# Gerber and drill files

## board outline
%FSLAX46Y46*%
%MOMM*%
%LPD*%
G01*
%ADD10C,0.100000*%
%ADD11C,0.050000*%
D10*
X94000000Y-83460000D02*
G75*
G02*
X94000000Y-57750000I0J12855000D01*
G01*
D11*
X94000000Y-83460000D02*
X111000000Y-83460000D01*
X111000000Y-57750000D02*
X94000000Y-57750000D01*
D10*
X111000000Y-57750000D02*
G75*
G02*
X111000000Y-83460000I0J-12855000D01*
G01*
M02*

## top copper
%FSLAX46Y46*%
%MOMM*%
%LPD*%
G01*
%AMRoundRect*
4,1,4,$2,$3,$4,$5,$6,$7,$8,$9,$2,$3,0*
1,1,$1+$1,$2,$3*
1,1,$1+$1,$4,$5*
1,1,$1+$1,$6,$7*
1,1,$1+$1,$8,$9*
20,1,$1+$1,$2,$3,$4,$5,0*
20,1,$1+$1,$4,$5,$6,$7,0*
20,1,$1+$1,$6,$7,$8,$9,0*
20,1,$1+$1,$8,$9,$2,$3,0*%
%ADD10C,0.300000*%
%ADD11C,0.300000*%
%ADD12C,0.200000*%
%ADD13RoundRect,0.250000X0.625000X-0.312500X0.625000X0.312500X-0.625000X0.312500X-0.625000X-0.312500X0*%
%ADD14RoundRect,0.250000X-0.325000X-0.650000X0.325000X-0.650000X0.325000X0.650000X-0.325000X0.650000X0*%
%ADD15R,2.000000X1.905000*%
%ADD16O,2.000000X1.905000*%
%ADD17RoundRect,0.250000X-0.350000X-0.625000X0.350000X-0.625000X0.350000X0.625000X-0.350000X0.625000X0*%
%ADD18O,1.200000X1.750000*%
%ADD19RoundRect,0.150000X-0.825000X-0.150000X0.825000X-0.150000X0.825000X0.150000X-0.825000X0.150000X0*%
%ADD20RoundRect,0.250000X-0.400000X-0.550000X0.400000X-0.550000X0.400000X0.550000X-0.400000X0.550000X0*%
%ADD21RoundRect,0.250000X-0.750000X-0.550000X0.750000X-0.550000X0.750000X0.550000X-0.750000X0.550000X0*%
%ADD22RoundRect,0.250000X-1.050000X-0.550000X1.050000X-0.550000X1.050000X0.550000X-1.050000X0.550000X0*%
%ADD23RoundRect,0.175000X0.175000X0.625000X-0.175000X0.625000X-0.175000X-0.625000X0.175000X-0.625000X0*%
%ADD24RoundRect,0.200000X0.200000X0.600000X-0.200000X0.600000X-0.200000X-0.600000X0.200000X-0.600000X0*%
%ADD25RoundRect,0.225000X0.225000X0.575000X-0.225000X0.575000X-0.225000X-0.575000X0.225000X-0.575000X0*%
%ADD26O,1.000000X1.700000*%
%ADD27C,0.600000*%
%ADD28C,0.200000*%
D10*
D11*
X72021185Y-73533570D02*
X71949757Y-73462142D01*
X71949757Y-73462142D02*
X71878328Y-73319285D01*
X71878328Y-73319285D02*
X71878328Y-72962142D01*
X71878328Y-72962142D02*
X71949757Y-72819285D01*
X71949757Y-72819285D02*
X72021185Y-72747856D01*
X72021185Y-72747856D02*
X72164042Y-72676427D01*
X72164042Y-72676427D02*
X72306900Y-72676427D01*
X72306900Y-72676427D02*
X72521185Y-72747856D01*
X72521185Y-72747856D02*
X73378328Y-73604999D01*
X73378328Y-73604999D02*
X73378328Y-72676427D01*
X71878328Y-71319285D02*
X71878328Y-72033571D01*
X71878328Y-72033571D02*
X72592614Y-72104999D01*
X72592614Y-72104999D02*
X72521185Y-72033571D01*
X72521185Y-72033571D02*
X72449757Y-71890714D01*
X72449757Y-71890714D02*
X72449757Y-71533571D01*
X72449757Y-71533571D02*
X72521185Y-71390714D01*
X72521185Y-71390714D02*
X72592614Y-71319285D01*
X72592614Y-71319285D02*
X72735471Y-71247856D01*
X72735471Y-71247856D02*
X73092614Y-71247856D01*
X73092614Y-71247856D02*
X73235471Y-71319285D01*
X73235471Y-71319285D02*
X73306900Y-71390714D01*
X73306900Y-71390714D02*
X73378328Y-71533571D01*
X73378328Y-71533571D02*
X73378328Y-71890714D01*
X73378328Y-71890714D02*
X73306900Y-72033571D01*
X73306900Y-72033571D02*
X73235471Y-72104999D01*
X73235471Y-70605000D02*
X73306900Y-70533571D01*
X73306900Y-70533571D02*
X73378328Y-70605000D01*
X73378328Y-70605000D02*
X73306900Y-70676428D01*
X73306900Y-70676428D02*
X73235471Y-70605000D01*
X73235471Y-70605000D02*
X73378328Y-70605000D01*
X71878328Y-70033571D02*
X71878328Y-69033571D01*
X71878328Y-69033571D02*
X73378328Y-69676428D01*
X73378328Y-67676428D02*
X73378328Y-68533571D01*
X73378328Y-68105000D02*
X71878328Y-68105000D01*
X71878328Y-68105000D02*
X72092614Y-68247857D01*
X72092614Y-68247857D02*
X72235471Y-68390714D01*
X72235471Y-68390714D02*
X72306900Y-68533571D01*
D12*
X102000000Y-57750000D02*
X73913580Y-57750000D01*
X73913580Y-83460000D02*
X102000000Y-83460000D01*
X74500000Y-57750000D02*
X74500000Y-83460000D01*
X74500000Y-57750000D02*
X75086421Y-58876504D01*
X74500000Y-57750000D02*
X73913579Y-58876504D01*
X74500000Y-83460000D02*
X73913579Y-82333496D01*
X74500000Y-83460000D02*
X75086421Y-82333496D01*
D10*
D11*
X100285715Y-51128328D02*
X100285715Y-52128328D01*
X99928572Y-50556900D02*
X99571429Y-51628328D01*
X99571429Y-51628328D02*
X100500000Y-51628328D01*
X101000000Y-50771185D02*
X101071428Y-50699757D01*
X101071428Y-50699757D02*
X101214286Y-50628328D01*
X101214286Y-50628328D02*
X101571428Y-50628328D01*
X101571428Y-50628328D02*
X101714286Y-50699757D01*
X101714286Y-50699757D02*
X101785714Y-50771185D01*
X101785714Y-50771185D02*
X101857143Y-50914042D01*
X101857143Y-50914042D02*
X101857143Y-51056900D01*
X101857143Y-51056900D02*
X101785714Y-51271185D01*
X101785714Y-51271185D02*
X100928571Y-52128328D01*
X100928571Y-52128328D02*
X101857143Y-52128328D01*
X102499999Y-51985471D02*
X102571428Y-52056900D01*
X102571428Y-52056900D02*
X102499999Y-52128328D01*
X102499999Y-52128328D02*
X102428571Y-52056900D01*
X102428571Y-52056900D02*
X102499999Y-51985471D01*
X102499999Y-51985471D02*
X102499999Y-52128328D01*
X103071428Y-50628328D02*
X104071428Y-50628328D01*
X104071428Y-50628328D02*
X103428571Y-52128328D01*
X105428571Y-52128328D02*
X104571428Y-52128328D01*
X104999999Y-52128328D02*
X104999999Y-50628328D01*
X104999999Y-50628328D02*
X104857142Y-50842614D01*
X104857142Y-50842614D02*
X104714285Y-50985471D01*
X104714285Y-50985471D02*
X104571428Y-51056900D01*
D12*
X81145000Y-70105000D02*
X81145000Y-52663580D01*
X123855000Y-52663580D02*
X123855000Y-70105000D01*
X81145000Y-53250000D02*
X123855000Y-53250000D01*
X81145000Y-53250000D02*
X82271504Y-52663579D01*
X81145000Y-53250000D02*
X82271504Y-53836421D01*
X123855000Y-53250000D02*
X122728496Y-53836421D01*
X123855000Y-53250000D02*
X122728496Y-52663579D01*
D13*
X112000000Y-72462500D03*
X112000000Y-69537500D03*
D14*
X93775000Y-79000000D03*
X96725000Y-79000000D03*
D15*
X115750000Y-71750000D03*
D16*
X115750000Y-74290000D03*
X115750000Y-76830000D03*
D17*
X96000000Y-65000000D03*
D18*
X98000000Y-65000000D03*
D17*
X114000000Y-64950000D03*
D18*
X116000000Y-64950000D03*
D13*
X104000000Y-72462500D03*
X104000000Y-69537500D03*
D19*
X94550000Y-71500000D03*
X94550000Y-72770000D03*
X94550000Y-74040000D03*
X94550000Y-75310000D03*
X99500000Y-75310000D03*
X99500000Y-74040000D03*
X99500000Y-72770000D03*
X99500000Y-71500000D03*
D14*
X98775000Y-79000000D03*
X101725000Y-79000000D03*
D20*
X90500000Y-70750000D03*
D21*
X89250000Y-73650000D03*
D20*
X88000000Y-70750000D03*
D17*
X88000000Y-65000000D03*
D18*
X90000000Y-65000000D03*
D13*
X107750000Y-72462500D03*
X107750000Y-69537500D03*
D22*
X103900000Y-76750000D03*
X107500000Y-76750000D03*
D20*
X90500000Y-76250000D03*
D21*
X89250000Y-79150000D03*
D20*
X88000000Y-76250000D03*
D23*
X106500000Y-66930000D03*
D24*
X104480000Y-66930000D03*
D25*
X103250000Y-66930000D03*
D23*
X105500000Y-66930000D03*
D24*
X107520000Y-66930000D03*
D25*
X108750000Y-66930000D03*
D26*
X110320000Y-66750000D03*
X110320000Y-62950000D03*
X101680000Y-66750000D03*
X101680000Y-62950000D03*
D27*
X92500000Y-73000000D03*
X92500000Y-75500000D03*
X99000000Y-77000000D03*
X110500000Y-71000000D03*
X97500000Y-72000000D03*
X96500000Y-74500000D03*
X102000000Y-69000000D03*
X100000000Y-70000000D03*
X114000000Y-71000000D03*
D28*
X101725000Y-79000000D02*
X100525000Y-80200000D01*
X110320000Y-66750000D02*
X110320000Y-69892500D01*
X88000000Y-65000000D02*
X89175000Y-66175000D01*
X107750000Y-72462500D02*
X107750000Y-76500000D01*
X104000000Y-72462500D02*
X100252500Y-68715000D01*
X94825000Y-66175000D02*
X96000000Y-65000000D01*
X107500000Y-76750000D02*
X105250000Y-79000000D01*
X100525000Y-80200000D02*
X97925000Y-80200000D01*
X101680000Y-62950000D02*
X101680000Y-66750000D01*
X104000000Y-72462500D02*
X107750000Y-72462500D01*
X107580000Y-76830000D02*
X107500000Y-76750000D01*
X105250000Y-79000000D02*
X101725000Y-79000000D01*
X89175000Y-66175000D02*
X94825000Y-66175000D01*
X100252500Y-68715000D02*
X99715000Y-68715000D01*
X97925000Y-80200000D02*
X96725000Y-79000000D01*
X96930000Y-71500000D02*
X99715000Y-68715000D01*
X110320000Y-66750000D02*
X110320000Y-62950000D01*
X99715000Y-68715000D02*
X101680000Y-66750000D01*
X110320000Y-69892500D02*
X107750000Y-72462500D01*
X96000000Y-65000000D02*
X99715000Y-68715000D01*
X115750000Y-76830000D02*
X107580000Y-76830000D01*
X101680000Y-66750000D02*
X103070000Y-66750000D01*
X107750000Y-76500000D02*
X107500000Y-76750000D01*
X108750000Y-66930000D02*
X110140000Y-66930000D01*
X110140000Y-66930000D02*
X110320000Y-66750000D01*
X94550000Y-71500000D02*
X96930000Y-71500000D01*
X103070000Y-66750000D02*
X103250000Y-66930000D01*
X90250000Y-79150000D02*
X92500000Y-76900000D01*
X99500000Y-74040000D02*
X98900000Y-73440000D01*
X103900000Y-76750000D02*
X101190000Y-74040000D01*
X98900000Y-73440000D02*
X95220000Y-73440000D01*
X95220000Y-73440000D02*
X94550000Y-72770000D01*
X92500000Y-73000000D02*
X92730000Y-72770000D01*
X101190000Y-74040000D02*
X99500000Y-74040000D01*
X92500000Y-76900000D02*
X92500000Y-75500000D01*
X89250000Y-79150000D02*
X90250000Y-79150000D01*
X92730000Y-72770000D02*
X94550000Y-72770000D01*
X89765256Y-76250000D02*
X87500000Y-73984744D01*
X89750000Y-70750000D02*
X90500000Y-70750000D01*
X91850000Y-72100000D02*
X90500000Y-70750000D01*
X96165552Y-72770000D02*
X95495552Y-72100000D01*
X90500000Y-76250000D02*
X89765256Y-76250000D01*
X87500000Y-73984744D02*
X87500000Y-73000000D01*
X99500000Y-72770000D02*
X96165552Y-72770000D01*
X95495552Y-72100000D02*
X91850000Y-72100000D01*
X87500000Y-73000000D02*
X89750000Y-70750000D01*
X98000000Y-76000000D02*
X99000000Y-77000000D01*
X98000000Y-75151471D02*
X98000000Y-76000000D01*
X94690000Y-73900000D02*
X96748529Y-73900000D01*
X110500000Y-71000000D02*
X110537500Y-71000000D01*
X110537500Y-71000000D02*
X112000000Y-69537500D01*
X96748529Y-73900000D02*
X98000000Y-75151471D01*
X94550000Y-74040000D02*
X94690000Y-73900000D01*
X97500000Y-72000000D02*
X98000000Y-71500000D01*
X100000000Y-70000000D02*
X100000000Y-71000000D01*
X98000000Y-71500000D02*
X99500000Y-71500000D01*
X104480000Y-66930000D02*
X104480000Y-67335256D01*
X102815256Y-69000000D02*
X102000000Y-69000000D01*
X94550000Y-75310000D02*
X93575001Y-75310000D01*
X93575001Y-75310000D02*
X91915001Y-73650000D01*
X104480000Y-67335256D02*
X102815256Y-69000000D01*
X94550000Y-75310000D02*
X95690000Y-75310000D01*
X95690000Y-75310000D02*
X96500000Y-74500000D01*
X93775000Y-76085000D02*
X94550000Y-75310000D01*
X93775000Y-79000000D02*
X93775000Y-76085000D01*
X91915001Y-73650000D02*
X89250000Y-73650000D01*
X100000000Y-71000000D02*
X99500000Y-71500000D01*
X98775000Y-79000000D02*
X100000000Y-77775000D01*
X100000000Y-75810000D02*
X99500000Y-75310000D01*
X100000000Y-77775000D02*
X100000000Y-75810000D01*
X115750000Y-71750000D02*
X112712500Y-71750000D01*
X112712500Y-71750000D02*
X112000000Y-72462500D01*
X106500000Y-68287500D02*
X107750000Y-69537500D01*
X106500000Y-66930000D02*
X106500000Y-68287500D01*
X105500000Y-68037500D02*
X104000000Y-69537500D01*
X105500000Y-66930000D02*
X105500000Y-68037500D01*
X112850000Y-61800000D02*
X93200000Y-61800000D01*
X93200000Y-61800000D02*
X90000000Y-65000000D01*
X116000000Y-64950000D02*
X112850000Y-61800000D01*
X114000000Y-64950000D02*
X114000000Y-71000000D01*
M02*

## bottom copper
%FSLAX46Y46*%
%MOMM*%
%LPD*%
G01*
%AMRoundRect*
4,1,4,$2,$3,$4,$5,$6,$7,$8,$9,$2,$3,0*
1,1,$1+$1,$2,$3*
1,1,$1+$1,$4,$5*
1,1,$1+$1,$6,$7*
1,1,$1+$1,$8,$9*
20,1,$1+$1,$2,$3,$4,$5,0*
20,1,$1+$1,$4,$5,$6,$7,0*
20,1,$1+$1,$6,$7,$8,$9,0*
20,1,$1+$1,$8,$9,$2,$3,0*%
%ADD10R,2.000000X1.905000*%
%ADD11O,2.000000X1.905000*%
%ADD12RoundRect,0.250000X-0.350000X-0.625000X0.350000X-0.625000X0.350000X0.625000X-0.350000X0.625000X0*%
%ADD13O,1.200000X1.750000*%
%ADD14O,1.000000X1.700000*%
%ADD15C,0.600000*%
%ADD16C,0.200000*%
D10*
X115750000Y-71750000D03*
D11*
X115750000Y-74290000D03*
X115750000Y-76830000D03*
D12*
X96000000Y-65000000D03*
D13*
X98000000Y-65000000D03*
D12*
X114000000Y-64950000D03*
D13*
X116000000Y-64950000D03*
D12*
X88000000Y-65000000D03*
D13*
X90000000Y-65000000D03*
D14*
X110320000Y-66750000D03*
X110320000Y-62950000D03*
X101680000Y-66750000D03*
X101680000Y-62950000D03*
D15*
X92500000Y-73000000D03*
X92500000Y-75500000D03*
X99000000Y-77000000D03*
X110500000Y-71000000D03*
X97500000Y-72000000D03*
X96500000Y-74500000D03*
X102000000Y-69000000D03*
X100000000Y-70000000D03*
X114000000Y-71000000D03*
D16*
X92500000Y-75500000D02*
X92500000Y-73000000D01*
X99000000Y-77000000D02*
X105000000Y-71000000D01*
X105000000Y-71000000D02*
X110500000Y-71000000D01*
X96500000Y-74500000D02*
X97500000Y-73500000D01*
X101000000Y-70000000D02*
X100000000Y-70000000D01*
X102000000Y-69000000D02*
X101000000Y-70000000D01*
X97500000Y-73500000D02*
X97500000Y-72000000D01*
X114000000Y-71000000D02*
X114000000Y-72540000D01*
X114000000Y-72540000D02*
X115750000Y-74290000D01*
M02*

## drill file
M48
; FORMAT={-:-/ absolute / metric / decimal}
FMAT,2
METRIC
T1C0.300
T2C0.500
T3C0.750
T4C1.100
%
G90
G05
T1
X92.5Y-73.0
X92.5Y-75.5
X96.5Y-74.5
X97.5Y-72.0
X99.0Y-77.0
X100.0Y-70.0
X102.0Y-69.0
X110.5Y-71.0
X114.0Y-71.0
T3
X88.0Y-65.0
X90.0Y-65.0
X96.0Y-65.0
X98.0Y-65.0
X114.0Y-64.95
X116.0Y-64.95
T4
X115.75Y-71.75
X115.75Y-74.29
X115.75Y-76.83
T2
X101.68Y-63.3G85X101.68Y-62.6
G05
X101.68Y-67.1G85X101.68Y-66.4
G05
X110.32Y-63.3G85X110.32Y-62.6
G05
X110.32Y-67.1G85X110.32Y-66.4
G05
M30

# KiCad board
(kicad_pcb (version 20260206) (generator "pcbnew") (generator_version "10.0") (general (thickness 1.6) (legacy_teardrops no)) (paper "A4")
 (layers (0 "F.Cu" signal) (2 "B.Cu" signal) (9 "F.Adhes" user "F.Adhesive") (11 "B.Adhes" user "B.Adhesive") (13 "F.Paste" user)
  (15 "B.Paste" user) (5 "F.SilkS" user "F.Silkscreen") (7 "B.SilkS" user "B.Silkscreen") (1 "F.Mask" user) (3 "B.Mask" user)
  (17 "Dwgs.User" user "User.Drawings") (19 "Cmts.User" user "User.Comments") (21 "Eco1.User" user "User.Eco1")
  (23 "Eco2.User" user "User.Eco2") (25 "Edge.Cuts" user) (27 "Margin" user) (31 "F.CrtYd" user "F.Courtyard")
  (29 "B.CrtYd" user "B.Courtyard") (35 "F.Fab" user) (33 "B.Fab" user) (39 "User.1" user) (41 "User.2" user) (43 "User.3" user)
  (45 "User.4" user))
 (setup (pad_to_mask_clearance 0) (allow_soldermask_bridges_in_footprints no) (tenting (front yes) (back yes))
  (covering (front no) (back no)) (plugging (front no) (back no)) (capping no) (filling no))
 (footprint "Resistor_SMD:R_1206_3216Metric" (layer "F.Cu") (at 112 71 90)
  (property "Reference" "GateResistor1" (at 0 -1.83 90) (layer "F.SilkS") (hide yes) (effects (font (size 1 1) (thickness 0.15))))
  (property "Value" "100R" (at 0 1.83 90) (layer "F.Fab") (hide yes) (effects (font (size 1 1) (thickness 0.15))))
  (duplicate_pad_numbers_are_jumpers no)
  (pad "1" smd roundrect (at -1.4625 0 90) (size 1.125 1.75) (layers "F.Cu" "F.Mask" "F.Paste") (roundrect_rratio 0.222222)
   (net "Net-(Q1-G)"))
  (pad "2" smd roundrect (at 1.4625 0 90) (size 1.125 1.75) (layers "F.Cu" "F.Mask" "F.Paste") (roundrect_rratio 0.222222) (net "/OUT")))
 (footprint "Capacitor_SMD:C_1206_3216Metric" (layer "F.Cu") (at 95.25 79)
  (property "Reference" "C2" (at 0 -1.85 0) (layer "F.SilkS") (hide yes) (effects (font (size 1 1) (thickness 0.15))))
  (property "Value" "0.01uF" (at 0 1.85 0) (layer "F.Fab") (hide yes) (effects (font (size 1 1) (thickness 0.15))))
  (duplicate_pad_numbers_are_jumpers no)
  (pad "1" smd roundrect (at -1.475 0) (size 1.15 1.8) (layers "F.Cu" "F.Mask" "F.Paste") (roundrect_rratio 0.217391) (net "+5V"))
  (pad "2" smd roundrect (at 1.475 0) (size 1.15 1.8) (layers "F.Cu" "F.Mask" "F.Paste") (roundrect_rratio 0.217391) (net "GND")))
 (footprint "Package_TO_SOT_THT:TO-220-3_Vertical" (layer "F.Cu") (at 115.75 71.75 -90)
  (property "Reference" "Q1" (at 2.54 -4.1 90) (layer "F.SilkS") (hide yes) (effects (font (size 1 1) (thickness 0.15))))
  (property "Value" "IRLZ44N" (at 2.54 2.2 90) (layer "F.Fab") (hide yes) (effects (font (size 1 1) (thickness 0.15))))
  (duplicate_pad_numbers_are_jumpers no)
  (pad "1" thru_hole rect (at 0 0 270) (size 1.905 2) (drill 1.1) (layers "*.Cu" "*.Mask") (remove_unused_layers no) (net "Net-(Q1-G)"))
  (pad "2" thru_hole oval (at 2.54 0 270) (size 1.905 2) (drill 1.1) (layers "*.Cu" "*.Mask") (remove_unused_layers no) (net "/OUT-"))
  (pad "3" thru_hole oval (at 5.08 0 270) (size 1.905 2) (drill 1.1) (layers "*.Cu" "*.Mask") (remove_unused_layers no) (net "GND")))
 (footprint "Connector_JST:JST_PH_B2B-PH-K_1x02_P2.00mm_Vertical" (layer "F.Cu") (at 96 65)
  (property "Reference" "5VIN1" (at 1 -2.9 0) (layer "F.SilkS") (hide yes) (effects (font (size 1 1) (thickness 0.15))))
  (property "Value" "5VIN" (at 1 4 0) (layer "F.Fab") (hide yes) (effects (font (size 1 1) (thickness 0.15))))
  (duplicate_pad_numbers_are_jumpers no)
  (pad "1" thru_hole roundrect (at 0 0) (size 1.2 1.75) (drill 0.75) (layers "*.Cu" "*.Mask") (remove_unused_layers no)
   (roundrect_rratio 0.208333) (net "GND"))
  (pad "2" thru_hole oval (at 2 0) (size 1.2 1.75) (drill 0.75) (layers "*.Cu" "*.Mask") (remove_unused_layers no) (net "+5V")))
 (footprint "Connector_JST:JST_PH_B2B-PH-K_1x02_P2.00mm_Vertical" (layer "F.Cu") (at 114 64.95)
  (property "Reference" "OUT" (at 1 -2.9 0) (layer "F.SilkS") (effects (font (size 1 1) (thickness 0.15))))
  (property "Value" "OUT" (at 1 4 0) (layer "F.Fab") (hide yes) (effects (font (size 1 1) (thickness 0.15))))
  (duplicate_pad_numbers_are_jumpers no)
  (pad "1" thru_hole roundrect (at 0 0) (size 1.2 1.75) (drill 0.75) (layers "*.Cu" "*.Mask") (remove_unused_layers no)
   (roundrect_rratio 0.208333) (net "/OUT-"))
  (pad "2" thru_hole oval (at 2 0) (size 1.2 1.75) (drill 0.75) (layers "*.Cu" "*.Mask") (remove_unused_layers no) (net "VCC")))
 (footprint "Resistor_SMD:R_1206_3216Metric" (layer "F.Cu") (at 104 71 90)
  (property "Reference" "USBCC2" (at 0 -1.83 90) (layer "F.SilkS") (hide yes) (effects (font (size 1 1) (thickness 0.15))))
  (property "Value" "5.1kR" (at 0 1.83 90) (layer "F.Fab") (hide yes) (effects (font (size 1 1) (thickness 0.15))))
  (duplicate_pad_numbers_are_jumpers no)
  (pad "1" smd roundrect (at -1.4625 0 90) (size 1.125 1.75) (layers "F.Cu" "F.Mask" "F.Paste") (roundrect_rratio 0.222222) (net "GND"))
  (pad "2" smd roundrect (at 1.4625 0 90) (size 1.125 1.75) (layers "F.Cu" "F.Mask" "F.Paste") (roundrect_rratio 0.222222) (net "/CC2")))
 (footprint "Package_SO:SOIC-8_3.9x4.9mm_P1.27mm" (layer "F.Cu") (at 97.025 73.405)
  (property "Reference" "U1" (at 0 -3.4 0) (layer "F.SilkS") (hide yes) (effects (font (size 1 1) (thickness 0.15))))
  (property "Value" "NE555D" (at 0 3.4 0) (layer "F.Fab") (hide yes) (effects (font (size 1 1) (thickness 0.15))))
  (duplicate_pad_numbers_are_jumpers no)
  (pad "1" smd roundrect (at -2.475 -1.905) (size 1.95 0.6) (layers "F.Cu" "F.Mask" "F.Paste") (roundrect_rratio 0.25) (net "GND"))
  (pad "2" smd roundrect (at -2.475 -0.635) (size 1.95 0.6) (layers "F.Cu" "F.Mask" "F.Paste") (roundrect_rratio 0.25) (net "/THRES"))
  (pad "3" smd roundrect (at -2.475 0.635) (size 1.95 0.6) (layers "F.Cu" "F.Mask" "F.Paste") (roundrect_rratio 0.25) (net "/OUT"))
  (pad "4" smd roundrect (at -2.475 1.905) (size 1.95 0.6) (layers "F.Cu" "F.Mask" "F.Paste") (roundrect_rratio 0.25) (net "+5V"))
  (pad "5" smd roundrect (at 2.475 1.905) (size 1.95 0.6) (layers "F.Cu" "F.Mask" "F.Paste") (roundrect_rratio 0.25) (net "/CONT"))
  (pad "6" smd roundrect (at 2.475 0.635) (size 1.95 0.6) (layers "F.Cu" "F.Mask" "F.Paste") (roundrect_rratio 0.25) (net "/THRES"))
  (pad "7" smd roundrect (at 2.475 -0.635) (size 1.95 0.6) (layers "F.Cu" "F.Mask" "F.Paste") (roundrect_rratio 0.25) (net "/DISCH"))
  (pad "8" smd roundrect (at 2.475 -1.905) (size 1.95 0.6) (layers "F.Cu" "F.Mask" "F.Paste") (roundrect_rratio 0.25) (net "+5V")))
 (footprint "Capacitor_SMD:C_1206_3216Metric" (layer "F.Cu") (at 100.25 79)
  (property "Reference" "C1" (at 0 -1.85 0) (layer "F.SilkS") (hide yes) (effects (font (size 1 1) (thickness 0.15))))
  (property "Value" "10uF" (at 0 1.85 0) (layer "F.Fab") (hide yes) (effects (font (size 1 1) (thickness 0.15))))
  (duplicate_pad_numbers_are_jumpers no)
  (pad "1" smd roundrect (at -1.475 0) (size 1.15 1.8) (layers "F.Cu" "F.Mask" "F.Paste") (roundrect_rratio 0.217391) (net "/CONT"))
  (pad "2" smd roundrect (at 1.475 0) (size 1.15 1.8) (layers "F.Cu" "F.Mask" "F.Paste") (roundrect_rratio 0.217391) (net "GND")))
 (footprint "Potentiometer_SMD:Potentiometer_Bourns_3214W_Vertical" (layer "F.Cu") (at 89.25 72.2)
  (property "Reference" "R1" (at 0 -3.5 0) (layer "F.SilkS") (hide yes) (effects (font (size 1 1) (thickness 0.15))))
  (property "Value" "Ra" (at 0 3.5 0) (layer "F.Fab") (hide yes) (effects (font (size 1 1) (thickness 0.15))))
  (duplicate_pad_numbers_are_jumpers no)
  (pad "1" smd roundrect (at 1.25 -1.45) (size 1.3 1.6) (layers "F.Cu" "F.Mask" "F.Paste") (roundrect_rratio 0.192308) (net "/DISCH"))
  (pad "2" smd roundrect (at 0 1.45) (size 2 1.6) (layers "F.Cu" "F.Mask" "F.Paste") (roundrect_rratio 0.15625) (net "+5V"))
  (pad "3" smd roundrect (at -1.25 -1.45) (size 1.3 1.6) (layers "F.Cu" "F.Mask" "F.Paste") (roundrect_rratio 0.192308)))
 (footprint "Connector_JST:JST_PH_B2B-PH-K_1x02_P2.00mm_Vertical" (layer "F.Cu") (at 88 65)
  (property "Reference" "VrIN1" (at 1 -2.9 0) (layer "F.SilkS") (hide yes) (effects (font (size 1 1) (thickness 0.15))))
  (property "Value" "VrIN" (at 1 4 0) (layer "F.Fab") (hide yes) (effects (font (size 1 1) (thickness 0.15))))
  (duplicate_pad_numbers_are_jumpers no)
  (pad "1" thru_hole roundrect (at 0 0) (size 1.2 1.75) (drill 0.75) (layers "*.Cu" "*.Mask") (remove_unused_layers no)
   (roundrect_rratio 0.208333) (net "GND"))
  (pad "2" thru_hole oval (at 2 0) (size 1.2 1.75) (drill 0.75) (layers "*.Cu" "*.Mask") (remove_unused_layers no) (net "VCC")))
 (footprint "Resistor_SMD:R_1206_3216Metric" (layer "F.Cu") (at 107.75 71 90)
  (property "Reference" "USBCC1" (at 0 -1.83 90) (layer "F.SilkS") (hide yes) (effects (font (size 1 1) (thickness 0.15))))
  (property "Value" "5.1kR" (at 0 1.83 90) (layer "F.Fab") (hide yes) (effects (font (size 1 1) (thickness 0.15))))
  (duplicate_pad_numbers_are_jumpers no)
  (pad "1" smd roundrect (at -1.4625 0 90) (size 1.125 1.75) (layers "F.Cu" "F.Mask" "F.Paste") (roundrect_rratio 0.222222) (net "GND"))
  (pad "2" smd roundrect (at 1.4625 0 90) (size 1.125 1.75) (layers "F.Cu" "F.Mask" "F.Paste") (roundrect_rratio 0.222222) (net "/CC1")))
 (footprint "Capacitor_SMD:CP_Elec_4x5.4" (layer "F.Cu") (at 105.7 76.75)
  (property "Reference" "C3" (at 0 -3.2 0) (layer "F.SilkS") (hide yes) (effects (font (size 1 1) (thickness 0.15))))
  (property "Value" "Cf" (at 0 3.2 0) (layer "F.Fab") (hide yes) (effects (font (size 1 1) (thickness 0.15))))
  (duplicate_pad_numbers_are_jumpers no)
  (pad "1" smd roundrect (at -1.8 0) (size 2.6 1.6) (layers "F.Cu" "F.Mask" "F.Paste") (roundrect_rratio 0.15625) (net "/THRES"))
  (pad "2" smd roundrect (at 1.8 0) (size 2.6 1.6) (layers "F.Cu" "F.Mask" "F.Paste") (roundrect_rratio 0.15625) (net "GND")))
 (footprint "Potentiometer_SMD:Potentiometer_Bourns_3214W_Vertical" (layer "F.Cu") (at 89.25 77.7)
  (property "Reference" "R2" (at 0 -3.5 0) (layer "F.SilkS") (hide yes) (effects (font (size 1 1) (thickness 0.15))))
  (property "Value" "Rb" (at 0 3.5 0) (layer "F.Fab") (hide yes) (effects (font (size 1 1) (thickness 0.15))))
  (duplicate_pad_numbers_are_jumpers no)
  (pad "1" smd roundrect (at 1.25 -1.45) (size 1.3 1.6) (layers "F.Cu" "F.Mask" "F.Paste") (roundrect_rratio 0.192308) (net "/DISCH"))
  (pad "2" smd roundrect (at 0 1.45) (size 2 1.6) (layers "F.Cu" "F.Mask" "F.Paste") (roundrect_rratio 0.15625) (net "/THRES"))
  (pad "3" smd roundrect (at -1.25 -1.45) (size 1.3 1.6) (layers "F.Cu" "F.Mask" "F.Paste") (roundrect_rratio 0.192308)))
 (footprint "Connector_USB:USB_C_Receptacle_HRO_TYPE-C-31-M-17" (layer "F.Cu") (at 106 63.75 180)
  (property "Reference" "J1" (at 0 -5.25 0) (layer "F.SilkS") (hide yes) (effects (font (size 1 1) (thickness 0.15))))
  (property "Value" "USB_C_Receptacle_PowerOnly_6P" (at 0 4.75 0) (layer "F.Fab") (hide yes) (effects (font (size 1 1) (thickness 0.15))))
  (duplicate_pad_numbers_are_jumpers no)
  (pad "A5" smd roundrect (at -0.5 -3.18 180) (size 0.7 1.6) (layers "F.Cu" "F.Mask" "F.Paste") (roundrect_rratio 0.25) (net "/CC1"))
  (pad "A9" smd roundrect (at 1.52 -3.18 180) (size 0.8 1.6) (layers "F.Cu" "F.Mask" "F.Paste") (roundrect_rratio 0.25) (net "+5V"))
  (pad "A12" smd roundrect (at 2.75 -3.18 180) (size 0.9 1.6) (layers "F.Cu" "F.Mask" "F.Paste") (roundrect_rratio 0.25) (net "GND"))
  (pad "B5" smd roundrect (at 0.5 -3.18 180) (size 0.7 1.6) (layers "F.Cu" "F.Mask" "F.Paste") (roundrect_rratio 0.25) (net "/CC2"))
  (pad "B9" smd roundrect (at -1.52 -3.18 180) (size 0.8 1.6) (layers "F.Cu" "F.Mask" "F.Paste") (roundrect_rratio 0.25) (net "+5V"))
  (pad "B12" smd roundrect (at -2.75 -3.18 180) (size 0.9 1.6) (layers "F.Cu" "F.Mask" "F.Paste") (roundrect_rratio 0.25) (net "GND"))
  (pad "S1" thru_hole oval (at -4.32 -3 180) (size 1 1.7) (drill oval 0.5 1.2) (layers "*.Cu" "*.Mask") (remove_unused_layers no)
   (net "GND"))
  (pad "S1" thru_hole oval (at -4.32 0.8 180) (size 1 1.7) (drill oval 0.5 1.2) (layers "*.Cu" "*.Mask") (remove_unused_layers no)
   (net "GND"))
  (pad "S1" thru_hole oval (at 4.32 -3 180) (size 1 1.7) (drill oval 0.5 1.2) (layers "*.Cu" "*.Mask") (remove_unused_layers no) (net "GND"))
  (pad "S1" thru_hole oval (at 4.32 0.8 180) (size 1 1.7) (drill oval 0.5 1.2) (layers "*.Cu" "*.Mask") (remove_unused_layers no)
   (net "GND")))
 (gr_arc (start 94 83.46) (mid 81.145 70.605) (end 94 57.75) (stroke (width 0.1) (type solid)) (layer "Edge.Cuts"))
 (gr_line (start 94 83.46) (end 111 83.46) (stroke (width 0.05) (type default)) (layer "Edge.Cuts"))
 (gr_line (start 111 57.75) (end 94 57.75) (stroke (width 0.05) (type default)) (layer "Edge.Cuts"))
 (gr_arc (start 111 57.75) (mid 123.855 70.605) (end 111 83.46) (stroke (width 0.1) (type solid)) (layer "Edge.Cuts"))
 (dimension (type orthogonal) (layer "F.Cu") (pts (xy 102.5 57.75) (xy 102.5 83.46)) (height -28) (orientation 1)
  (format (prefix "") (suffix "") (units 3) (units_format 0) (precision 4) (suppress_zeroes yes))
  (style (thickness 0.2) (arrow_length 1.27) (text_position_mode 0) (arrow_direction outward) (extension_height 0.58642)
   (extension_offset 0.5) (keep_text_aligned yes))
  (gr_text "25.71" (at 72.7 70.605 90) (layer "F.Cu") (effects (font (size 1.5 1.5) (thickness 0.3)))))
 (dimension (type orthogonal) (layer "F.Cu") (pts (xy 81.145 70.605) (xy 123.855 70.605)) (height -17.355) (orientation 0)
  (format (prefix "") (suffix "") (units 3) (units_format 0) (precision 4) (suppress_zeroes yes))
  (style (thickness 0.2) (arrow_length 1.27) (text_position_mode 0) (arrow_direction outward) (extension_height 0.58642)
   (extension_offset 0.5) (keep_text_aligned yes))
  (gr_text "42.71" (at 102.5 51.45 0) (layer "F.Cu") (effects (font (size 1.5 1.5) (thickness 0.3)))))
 (segment (start 101.725 79) (end 100.525 80.2) (width 0.2) (layer "F.Cu") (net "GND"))
 (segment (start 110.32 66.75) (end 110.32 69.8925) (width 0.2) (layer "F.Cu") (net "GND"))
 (segment (start 88 65) (end 89.175 66.175) (width 0.2) (layer "F.Cu") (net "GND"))
 (segment (start 107.75 72.4625) (end 107.75 76.5) (width 0.2) (layer "F.Cu") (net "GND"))
 (segment (start 104 72.4625) (end 100.2525 68.715) (width 0.2) (layer "F.Cu") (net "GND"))
 (segment (start 94.825 66.175) (end 96 65) (width 0.2) (layer "F.Cu") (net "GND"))
 (segment (start 107.5 76.75) (end 105.25 79) (width 0.2) (layer "F.Cu") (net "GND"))
 (segment (start 100.525 80.2) (end 97.925 80.2) (width 0.2) (layer "F.Cu") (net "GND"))
 (segment (start 101.68 62.95) (end 101.68 66.75) (width 0.2) (layer "F.Cu") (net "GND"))
 (segment (start 104 72.4625) (end 107.75 72.4625) (width 0.2) (layer "F.Cu") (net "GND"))
 (segment (start 107.58 76.83) (end 107.5 76.75) (width 0.2) (layer "F.Cu") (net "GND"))
 (segment (start 105.25 79) (end 101.725 79) (width 0.2) (layer "F.Cu") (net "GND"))
 (segment (start 89.175 66.175) (end 94.825 66.175) (width 0.2) (layer "F.Cu") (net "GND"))
 (segment (start 100.2525 68.715) (end 99.715 68.715) (width 0.2) (layer "F.Cu") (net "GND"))
 (segment (start 97.925 80.2) (end 96.725 79) (width 0.2) (layer "F.Cu") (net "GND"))
 (segment (start 96.93 71.5) (end 99.715 68.715) (width 0.2) (layer "F.Cu") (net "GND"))
 (segment (start 110.32 66.75) (end 110.32 62.95) (width 0.2) (layer "F.Cu") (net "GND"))
 (segment (start 99.715 68.715) (end 101.68 66.75) (width 0.2) (layer "F.Cu") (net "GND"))
 (segment (start 110.32 69.8925) (end 107.75 72.4625) (width 0.2) (layer "F.Cu") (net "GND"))
 (segment (start 96 65) (end 99.715 68.715) (width 0.2) (layer "F.Cu") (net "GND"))
 (segment (start 115.75 76.83) (end 107.58 76.83) (width 0.2) (layer "F.Cu") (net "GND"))
 (segment (start 101.68 66.75) (end 103.07 66.75) (width 0.2) (layer "F.Cu") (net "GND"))
 (segment (start 107.75 76.5) (end 107.5 76.75) (width 0.2) (layer "F.Cu") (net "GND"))
 (segment (start 108.75 66.93) (end 110.14 66.93) (width 0.2) (layer "F.Cu") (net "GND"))
 (segment (start 110.14 66.93) (end 110.32 66.75) (width 0.2) (layer "F.Cu") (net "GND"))
 (segment (start 94.55 71.5) (end 96.93 71.5) (width 0.2) (layer "F.Cu") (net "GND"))
 (segment (start 103.07 66.75) (end 103.25 66.93) (width 0.2) (layer "F.Cu") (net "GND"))
 (segment (start 90.25 79.15) (end 92.5 76.9) (width 0.2) (layer "F.Cu") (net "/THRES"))
 (segment (start 99.5 74.04) (end 98.9 73.44) (width 0.2) (layer "F.Cu") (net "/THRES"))
 (segment (start 103.9 76.75) (end 101.19 74.04) (width 0.2) (layer "F.Cu") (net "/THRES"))
 (segment (start 98.9 73.44) (end 95.22 73.44) (width 0.2) (layer "F.Cu") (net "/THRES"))
 (segment (start 95.22 73.44) (end 94.55 72.77) (width 0.2) (layer "F.Cu") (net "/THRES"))
 (segment (start 92.5 73) (end 92.73 72.77) (width 0.2) (layer "F.Cu") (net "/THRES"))
 (segment (start 101.19 74.04) (end 99.5 74.04) (width 0.2) (layer "F.Cu") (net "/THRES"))
 (segment (start 92.5 76.9) (end 92.5 75.5) (width 0.2) (layer "F.Cu") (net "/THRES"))
 (segment (start 89.25 79.15) (end 90.25 79.15) (width 0.2) (layer "F.Cu") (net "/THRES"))
 (segment (start 92.73 72.77) (end 94.55 72.77) (width 0.2) (layer "F.Cu") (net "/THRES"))
 (via (at 92.5 73) (size 0.6) (drill 0.3) (layers "F.Cu" "B.Cu") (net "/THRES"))
 (via (at 92.5 75.5) (size 0.6) (drill 0.3) (layers "F.Cu" "B.Cu") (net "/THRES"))
 (segment (start 92.5 75.5) (end 92.5 73) (width 0.2) (layer "B.Cu") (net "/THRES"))
 (segment (start 89.765256 76.25) (end 87.5 73.984744) (width 0.2) (layer "F.Cu") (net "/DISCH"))
 (segment (start 89.75 70.75) (end 90.5 70.75) (width 0.2) (layer "F.Cu") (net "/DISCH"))
 (segment (start 91.85 72.1) (end 90.5 70.75) (width 0.2) (layer "F.Cu") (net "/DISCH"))
 (segment (start 96.165552 72.77) (end 95.495552 72.1) (width 0.2) (layer "F.Cu") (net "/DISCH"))
 (segment (start 90.5 76.25) (end 89.765256 76.25) (width 0.2) (layer "F.Cu") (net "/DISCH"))
 (segment (start 87.5 73.984744) (end 87.5 73) (width 0.2) (layer "F.Cu") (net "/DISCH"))
 (segment (start 99.5 72.77) (end 96.165552 72.77) (width 0.2) (layer "F.Cu") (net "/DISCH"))
 (segment (start 95.495552 72.1) (end 91.85 72.1) (width 0.2) (layer "F.Cu") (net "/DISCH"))
 (segment (start 87.5 73) (end 89.75 70.75) (width 0.2) (layer "F.Cu") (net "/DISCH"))
 (segment (start 98 76) (end 99 77) (width 0.2) (layer "F.Cu") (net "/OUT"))
 (segment (start 98 75.151471) (end 98 76) (width 0.2) (layer "F.Cu") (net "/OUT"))
 (segment (start 94.69 73.9) (end 96.748529 73.9) (width 0.2) (layer "F.Cu") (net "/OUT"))
 (segment (start 110.5 71) (end 110.5375 71) (width 0.2) (layer "F.Cu") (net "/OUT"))
 (segment (start 110.5375 71) (end 112 69.5375) (width 0.2) (layer "F.Cu") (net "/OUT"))
 (segment (start 96.748529 73.9) (end 98 75.151471) (width 0.2) (layer "F.Cu") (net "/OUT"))
 (segment (start 94.55 74.04) (end 94.69 73.9) (width 0.2) (layer "F.Cu") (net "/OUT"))
 (via (at 99 77) (size 0.6) (drill 0.3) (layers "F.Cu" "B.Cu") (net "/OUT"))
 (via (at 110.5 71) (size 0.6) (drill 0.3) (layers "F.Cu" "B.Cu") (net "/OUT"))
 (segment (start 99 77) (end 105 71) (width 0.2) (layer "B.Cu") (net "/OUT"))
 (segment (start 105 71) (end 110.5 71) (width 0.2) (layer "B.Cu") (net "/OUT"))
 (segment (start 97.5 72) (end 98 71.5) (width 0.2) (layer "F.Cu") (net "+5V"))
 (segment (start 100 70) (end 100 71) (width 0.2) (layer "F.Cu") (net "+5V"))
 (segment (start 98 71.5) (end 99.5 71.5) (width 0.2) (layer "F.Cu") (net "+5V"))
 (segment (start 104.48 66.93) (end 104.48 67.335256) (width 0.2) (layer "F.Cu") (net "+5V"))
 (segment (start 102.815256 69) (end 102 69) (width 0.2) (layer "F.Cu") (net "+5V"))
 (segment (start 94.55 75.31) (end 93.575001 75.31) (width 0.2) (layer "F.Cu") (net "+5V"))
 (segment (start 93.575001 75.31) (end 91.915001 73.65) (width 0.2) (layer "F.Cu") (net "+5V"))
 (segment (start 104.48 67.335256) (end 102.815256 69) (width 0.2) (layer "F.Cu") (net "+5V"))
 (segment (start 94.55 75.31) (end 95.69 75.31) (width 0.2) (layer "F.Cu") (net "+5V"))
 (segment (start 95.69 75.31) (end 96.5 74.5) (width 0.2) (layer "F.Cu") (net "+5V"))
 (segment (start 93.775 76.085) (end 94.55 75.31) (width 0.2) (layer "F.Cu") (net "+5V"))
 (segment (start 93.775 79) (end 93.775 76.085) (width 0.2) (layer "F.Cu") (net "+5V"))
 (segment (start 91.915001 73.65) (end 89.25 73.65) (width 0.2) (layer "F.Cu") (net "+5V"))
 (segment (start 100 71) (end 99.5 71.5) (width 0.2) (layer "F.Cu") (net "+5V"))
 (via (at 97.5 72) (size 0.6) (drill 0.3) (layers "F.Cu" "B.Cu") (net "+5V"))
 (via (at 96.5 74.5) (size 0.6) (drill 0.3) (layers "F.Cu" "B.Cu") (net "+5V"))
 (via (at 102 69) (size 0.6) (drill 0.3) (layers "F.Cu" "B.Cu") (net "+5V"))
 (via (at 100 70) (size 0.6) (drill 0.3) (layers "F.Cu" "B.Cu") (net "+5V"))
 (segment (start 96.5 74.5) (end 97.5 73.5) (width 0.2) (layer "B.Cu") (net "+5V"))
 (segment (start 101 70) (end 100 70) (width 0.2) (layer "B.Cu") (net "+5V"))
 (segment (start 102 69) (end 101 70) (width 0.2) (layer "B.Cu") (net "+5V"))
 (segment (start 97.5 73.5) (end 97.5 72) (width 0.2) (layer "B.Cu") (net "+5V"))
 (segment (start 98.775 79) (end 100 77.775) (width 0.2) (layer "F.Cu") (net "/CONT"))
 (segment (start 100 75.81) (end 99.5 75.31) (width 0.2) (layer "F.Cu") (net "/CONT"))
 (segment (start 100 77.775) (end 100 75.81) (width 0.2) (layer "F.Cu") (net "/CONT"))
 (segment (start 115.75 71.75) (end 112.7125 71.75) (width 0.2) (layer "F.Cu") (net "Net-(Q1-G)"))
 (segment (start 112.7125 71.75) (end 112 72.4625) (width 0.2) (layer "F.Cu") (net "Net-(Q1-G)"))
 (segment (start 106.5 68.2875) (end 107.75 69.5375) (width 0.2) (layer "F.Cu") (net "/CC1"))
 (segment (start 106.5 66.93) (end 106.5 68.2875) (width 0.2) (layer "F.Cu") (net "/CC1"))
 (segment (start 105.5 68.0375) (end 104 69.5375) (width 0.2) (layer "F.Cu") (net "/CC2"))
 (segment (start 105.5 66.93) (end 105.5 68.0375) (width 0.2) (layer "F.Cu") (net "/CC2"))
 (segment (start 112.85 61.8) (end 93.2 61.8) (width 0.2) (layer "F.Cu") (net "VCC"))
 (segment (start 93.2 61.8) (end 90 65) (width 0.2) (layer "F.Cu") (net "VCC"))
 (segment (start 116 64.95) (end 112.85 61.8) (width 0.2) (layer "F.Cu") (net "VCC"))
 (segment (start 114 64.95) (end 114 71) (width 0.2) (layer "F.Cu") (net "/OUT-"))
 (via (at 114 71) (size 0.6) (drill 0.3) (layers "F.Cu" "B.Cu") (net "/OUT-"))
 (segment (start 114 71) (end 114 72.54) (width 0.2) (layer "B.Cu") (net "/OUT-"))
 (segment (start 114 72.54) (end 115.75 74.29) (width 0.2) (layer "B.Cu") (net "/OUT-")))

